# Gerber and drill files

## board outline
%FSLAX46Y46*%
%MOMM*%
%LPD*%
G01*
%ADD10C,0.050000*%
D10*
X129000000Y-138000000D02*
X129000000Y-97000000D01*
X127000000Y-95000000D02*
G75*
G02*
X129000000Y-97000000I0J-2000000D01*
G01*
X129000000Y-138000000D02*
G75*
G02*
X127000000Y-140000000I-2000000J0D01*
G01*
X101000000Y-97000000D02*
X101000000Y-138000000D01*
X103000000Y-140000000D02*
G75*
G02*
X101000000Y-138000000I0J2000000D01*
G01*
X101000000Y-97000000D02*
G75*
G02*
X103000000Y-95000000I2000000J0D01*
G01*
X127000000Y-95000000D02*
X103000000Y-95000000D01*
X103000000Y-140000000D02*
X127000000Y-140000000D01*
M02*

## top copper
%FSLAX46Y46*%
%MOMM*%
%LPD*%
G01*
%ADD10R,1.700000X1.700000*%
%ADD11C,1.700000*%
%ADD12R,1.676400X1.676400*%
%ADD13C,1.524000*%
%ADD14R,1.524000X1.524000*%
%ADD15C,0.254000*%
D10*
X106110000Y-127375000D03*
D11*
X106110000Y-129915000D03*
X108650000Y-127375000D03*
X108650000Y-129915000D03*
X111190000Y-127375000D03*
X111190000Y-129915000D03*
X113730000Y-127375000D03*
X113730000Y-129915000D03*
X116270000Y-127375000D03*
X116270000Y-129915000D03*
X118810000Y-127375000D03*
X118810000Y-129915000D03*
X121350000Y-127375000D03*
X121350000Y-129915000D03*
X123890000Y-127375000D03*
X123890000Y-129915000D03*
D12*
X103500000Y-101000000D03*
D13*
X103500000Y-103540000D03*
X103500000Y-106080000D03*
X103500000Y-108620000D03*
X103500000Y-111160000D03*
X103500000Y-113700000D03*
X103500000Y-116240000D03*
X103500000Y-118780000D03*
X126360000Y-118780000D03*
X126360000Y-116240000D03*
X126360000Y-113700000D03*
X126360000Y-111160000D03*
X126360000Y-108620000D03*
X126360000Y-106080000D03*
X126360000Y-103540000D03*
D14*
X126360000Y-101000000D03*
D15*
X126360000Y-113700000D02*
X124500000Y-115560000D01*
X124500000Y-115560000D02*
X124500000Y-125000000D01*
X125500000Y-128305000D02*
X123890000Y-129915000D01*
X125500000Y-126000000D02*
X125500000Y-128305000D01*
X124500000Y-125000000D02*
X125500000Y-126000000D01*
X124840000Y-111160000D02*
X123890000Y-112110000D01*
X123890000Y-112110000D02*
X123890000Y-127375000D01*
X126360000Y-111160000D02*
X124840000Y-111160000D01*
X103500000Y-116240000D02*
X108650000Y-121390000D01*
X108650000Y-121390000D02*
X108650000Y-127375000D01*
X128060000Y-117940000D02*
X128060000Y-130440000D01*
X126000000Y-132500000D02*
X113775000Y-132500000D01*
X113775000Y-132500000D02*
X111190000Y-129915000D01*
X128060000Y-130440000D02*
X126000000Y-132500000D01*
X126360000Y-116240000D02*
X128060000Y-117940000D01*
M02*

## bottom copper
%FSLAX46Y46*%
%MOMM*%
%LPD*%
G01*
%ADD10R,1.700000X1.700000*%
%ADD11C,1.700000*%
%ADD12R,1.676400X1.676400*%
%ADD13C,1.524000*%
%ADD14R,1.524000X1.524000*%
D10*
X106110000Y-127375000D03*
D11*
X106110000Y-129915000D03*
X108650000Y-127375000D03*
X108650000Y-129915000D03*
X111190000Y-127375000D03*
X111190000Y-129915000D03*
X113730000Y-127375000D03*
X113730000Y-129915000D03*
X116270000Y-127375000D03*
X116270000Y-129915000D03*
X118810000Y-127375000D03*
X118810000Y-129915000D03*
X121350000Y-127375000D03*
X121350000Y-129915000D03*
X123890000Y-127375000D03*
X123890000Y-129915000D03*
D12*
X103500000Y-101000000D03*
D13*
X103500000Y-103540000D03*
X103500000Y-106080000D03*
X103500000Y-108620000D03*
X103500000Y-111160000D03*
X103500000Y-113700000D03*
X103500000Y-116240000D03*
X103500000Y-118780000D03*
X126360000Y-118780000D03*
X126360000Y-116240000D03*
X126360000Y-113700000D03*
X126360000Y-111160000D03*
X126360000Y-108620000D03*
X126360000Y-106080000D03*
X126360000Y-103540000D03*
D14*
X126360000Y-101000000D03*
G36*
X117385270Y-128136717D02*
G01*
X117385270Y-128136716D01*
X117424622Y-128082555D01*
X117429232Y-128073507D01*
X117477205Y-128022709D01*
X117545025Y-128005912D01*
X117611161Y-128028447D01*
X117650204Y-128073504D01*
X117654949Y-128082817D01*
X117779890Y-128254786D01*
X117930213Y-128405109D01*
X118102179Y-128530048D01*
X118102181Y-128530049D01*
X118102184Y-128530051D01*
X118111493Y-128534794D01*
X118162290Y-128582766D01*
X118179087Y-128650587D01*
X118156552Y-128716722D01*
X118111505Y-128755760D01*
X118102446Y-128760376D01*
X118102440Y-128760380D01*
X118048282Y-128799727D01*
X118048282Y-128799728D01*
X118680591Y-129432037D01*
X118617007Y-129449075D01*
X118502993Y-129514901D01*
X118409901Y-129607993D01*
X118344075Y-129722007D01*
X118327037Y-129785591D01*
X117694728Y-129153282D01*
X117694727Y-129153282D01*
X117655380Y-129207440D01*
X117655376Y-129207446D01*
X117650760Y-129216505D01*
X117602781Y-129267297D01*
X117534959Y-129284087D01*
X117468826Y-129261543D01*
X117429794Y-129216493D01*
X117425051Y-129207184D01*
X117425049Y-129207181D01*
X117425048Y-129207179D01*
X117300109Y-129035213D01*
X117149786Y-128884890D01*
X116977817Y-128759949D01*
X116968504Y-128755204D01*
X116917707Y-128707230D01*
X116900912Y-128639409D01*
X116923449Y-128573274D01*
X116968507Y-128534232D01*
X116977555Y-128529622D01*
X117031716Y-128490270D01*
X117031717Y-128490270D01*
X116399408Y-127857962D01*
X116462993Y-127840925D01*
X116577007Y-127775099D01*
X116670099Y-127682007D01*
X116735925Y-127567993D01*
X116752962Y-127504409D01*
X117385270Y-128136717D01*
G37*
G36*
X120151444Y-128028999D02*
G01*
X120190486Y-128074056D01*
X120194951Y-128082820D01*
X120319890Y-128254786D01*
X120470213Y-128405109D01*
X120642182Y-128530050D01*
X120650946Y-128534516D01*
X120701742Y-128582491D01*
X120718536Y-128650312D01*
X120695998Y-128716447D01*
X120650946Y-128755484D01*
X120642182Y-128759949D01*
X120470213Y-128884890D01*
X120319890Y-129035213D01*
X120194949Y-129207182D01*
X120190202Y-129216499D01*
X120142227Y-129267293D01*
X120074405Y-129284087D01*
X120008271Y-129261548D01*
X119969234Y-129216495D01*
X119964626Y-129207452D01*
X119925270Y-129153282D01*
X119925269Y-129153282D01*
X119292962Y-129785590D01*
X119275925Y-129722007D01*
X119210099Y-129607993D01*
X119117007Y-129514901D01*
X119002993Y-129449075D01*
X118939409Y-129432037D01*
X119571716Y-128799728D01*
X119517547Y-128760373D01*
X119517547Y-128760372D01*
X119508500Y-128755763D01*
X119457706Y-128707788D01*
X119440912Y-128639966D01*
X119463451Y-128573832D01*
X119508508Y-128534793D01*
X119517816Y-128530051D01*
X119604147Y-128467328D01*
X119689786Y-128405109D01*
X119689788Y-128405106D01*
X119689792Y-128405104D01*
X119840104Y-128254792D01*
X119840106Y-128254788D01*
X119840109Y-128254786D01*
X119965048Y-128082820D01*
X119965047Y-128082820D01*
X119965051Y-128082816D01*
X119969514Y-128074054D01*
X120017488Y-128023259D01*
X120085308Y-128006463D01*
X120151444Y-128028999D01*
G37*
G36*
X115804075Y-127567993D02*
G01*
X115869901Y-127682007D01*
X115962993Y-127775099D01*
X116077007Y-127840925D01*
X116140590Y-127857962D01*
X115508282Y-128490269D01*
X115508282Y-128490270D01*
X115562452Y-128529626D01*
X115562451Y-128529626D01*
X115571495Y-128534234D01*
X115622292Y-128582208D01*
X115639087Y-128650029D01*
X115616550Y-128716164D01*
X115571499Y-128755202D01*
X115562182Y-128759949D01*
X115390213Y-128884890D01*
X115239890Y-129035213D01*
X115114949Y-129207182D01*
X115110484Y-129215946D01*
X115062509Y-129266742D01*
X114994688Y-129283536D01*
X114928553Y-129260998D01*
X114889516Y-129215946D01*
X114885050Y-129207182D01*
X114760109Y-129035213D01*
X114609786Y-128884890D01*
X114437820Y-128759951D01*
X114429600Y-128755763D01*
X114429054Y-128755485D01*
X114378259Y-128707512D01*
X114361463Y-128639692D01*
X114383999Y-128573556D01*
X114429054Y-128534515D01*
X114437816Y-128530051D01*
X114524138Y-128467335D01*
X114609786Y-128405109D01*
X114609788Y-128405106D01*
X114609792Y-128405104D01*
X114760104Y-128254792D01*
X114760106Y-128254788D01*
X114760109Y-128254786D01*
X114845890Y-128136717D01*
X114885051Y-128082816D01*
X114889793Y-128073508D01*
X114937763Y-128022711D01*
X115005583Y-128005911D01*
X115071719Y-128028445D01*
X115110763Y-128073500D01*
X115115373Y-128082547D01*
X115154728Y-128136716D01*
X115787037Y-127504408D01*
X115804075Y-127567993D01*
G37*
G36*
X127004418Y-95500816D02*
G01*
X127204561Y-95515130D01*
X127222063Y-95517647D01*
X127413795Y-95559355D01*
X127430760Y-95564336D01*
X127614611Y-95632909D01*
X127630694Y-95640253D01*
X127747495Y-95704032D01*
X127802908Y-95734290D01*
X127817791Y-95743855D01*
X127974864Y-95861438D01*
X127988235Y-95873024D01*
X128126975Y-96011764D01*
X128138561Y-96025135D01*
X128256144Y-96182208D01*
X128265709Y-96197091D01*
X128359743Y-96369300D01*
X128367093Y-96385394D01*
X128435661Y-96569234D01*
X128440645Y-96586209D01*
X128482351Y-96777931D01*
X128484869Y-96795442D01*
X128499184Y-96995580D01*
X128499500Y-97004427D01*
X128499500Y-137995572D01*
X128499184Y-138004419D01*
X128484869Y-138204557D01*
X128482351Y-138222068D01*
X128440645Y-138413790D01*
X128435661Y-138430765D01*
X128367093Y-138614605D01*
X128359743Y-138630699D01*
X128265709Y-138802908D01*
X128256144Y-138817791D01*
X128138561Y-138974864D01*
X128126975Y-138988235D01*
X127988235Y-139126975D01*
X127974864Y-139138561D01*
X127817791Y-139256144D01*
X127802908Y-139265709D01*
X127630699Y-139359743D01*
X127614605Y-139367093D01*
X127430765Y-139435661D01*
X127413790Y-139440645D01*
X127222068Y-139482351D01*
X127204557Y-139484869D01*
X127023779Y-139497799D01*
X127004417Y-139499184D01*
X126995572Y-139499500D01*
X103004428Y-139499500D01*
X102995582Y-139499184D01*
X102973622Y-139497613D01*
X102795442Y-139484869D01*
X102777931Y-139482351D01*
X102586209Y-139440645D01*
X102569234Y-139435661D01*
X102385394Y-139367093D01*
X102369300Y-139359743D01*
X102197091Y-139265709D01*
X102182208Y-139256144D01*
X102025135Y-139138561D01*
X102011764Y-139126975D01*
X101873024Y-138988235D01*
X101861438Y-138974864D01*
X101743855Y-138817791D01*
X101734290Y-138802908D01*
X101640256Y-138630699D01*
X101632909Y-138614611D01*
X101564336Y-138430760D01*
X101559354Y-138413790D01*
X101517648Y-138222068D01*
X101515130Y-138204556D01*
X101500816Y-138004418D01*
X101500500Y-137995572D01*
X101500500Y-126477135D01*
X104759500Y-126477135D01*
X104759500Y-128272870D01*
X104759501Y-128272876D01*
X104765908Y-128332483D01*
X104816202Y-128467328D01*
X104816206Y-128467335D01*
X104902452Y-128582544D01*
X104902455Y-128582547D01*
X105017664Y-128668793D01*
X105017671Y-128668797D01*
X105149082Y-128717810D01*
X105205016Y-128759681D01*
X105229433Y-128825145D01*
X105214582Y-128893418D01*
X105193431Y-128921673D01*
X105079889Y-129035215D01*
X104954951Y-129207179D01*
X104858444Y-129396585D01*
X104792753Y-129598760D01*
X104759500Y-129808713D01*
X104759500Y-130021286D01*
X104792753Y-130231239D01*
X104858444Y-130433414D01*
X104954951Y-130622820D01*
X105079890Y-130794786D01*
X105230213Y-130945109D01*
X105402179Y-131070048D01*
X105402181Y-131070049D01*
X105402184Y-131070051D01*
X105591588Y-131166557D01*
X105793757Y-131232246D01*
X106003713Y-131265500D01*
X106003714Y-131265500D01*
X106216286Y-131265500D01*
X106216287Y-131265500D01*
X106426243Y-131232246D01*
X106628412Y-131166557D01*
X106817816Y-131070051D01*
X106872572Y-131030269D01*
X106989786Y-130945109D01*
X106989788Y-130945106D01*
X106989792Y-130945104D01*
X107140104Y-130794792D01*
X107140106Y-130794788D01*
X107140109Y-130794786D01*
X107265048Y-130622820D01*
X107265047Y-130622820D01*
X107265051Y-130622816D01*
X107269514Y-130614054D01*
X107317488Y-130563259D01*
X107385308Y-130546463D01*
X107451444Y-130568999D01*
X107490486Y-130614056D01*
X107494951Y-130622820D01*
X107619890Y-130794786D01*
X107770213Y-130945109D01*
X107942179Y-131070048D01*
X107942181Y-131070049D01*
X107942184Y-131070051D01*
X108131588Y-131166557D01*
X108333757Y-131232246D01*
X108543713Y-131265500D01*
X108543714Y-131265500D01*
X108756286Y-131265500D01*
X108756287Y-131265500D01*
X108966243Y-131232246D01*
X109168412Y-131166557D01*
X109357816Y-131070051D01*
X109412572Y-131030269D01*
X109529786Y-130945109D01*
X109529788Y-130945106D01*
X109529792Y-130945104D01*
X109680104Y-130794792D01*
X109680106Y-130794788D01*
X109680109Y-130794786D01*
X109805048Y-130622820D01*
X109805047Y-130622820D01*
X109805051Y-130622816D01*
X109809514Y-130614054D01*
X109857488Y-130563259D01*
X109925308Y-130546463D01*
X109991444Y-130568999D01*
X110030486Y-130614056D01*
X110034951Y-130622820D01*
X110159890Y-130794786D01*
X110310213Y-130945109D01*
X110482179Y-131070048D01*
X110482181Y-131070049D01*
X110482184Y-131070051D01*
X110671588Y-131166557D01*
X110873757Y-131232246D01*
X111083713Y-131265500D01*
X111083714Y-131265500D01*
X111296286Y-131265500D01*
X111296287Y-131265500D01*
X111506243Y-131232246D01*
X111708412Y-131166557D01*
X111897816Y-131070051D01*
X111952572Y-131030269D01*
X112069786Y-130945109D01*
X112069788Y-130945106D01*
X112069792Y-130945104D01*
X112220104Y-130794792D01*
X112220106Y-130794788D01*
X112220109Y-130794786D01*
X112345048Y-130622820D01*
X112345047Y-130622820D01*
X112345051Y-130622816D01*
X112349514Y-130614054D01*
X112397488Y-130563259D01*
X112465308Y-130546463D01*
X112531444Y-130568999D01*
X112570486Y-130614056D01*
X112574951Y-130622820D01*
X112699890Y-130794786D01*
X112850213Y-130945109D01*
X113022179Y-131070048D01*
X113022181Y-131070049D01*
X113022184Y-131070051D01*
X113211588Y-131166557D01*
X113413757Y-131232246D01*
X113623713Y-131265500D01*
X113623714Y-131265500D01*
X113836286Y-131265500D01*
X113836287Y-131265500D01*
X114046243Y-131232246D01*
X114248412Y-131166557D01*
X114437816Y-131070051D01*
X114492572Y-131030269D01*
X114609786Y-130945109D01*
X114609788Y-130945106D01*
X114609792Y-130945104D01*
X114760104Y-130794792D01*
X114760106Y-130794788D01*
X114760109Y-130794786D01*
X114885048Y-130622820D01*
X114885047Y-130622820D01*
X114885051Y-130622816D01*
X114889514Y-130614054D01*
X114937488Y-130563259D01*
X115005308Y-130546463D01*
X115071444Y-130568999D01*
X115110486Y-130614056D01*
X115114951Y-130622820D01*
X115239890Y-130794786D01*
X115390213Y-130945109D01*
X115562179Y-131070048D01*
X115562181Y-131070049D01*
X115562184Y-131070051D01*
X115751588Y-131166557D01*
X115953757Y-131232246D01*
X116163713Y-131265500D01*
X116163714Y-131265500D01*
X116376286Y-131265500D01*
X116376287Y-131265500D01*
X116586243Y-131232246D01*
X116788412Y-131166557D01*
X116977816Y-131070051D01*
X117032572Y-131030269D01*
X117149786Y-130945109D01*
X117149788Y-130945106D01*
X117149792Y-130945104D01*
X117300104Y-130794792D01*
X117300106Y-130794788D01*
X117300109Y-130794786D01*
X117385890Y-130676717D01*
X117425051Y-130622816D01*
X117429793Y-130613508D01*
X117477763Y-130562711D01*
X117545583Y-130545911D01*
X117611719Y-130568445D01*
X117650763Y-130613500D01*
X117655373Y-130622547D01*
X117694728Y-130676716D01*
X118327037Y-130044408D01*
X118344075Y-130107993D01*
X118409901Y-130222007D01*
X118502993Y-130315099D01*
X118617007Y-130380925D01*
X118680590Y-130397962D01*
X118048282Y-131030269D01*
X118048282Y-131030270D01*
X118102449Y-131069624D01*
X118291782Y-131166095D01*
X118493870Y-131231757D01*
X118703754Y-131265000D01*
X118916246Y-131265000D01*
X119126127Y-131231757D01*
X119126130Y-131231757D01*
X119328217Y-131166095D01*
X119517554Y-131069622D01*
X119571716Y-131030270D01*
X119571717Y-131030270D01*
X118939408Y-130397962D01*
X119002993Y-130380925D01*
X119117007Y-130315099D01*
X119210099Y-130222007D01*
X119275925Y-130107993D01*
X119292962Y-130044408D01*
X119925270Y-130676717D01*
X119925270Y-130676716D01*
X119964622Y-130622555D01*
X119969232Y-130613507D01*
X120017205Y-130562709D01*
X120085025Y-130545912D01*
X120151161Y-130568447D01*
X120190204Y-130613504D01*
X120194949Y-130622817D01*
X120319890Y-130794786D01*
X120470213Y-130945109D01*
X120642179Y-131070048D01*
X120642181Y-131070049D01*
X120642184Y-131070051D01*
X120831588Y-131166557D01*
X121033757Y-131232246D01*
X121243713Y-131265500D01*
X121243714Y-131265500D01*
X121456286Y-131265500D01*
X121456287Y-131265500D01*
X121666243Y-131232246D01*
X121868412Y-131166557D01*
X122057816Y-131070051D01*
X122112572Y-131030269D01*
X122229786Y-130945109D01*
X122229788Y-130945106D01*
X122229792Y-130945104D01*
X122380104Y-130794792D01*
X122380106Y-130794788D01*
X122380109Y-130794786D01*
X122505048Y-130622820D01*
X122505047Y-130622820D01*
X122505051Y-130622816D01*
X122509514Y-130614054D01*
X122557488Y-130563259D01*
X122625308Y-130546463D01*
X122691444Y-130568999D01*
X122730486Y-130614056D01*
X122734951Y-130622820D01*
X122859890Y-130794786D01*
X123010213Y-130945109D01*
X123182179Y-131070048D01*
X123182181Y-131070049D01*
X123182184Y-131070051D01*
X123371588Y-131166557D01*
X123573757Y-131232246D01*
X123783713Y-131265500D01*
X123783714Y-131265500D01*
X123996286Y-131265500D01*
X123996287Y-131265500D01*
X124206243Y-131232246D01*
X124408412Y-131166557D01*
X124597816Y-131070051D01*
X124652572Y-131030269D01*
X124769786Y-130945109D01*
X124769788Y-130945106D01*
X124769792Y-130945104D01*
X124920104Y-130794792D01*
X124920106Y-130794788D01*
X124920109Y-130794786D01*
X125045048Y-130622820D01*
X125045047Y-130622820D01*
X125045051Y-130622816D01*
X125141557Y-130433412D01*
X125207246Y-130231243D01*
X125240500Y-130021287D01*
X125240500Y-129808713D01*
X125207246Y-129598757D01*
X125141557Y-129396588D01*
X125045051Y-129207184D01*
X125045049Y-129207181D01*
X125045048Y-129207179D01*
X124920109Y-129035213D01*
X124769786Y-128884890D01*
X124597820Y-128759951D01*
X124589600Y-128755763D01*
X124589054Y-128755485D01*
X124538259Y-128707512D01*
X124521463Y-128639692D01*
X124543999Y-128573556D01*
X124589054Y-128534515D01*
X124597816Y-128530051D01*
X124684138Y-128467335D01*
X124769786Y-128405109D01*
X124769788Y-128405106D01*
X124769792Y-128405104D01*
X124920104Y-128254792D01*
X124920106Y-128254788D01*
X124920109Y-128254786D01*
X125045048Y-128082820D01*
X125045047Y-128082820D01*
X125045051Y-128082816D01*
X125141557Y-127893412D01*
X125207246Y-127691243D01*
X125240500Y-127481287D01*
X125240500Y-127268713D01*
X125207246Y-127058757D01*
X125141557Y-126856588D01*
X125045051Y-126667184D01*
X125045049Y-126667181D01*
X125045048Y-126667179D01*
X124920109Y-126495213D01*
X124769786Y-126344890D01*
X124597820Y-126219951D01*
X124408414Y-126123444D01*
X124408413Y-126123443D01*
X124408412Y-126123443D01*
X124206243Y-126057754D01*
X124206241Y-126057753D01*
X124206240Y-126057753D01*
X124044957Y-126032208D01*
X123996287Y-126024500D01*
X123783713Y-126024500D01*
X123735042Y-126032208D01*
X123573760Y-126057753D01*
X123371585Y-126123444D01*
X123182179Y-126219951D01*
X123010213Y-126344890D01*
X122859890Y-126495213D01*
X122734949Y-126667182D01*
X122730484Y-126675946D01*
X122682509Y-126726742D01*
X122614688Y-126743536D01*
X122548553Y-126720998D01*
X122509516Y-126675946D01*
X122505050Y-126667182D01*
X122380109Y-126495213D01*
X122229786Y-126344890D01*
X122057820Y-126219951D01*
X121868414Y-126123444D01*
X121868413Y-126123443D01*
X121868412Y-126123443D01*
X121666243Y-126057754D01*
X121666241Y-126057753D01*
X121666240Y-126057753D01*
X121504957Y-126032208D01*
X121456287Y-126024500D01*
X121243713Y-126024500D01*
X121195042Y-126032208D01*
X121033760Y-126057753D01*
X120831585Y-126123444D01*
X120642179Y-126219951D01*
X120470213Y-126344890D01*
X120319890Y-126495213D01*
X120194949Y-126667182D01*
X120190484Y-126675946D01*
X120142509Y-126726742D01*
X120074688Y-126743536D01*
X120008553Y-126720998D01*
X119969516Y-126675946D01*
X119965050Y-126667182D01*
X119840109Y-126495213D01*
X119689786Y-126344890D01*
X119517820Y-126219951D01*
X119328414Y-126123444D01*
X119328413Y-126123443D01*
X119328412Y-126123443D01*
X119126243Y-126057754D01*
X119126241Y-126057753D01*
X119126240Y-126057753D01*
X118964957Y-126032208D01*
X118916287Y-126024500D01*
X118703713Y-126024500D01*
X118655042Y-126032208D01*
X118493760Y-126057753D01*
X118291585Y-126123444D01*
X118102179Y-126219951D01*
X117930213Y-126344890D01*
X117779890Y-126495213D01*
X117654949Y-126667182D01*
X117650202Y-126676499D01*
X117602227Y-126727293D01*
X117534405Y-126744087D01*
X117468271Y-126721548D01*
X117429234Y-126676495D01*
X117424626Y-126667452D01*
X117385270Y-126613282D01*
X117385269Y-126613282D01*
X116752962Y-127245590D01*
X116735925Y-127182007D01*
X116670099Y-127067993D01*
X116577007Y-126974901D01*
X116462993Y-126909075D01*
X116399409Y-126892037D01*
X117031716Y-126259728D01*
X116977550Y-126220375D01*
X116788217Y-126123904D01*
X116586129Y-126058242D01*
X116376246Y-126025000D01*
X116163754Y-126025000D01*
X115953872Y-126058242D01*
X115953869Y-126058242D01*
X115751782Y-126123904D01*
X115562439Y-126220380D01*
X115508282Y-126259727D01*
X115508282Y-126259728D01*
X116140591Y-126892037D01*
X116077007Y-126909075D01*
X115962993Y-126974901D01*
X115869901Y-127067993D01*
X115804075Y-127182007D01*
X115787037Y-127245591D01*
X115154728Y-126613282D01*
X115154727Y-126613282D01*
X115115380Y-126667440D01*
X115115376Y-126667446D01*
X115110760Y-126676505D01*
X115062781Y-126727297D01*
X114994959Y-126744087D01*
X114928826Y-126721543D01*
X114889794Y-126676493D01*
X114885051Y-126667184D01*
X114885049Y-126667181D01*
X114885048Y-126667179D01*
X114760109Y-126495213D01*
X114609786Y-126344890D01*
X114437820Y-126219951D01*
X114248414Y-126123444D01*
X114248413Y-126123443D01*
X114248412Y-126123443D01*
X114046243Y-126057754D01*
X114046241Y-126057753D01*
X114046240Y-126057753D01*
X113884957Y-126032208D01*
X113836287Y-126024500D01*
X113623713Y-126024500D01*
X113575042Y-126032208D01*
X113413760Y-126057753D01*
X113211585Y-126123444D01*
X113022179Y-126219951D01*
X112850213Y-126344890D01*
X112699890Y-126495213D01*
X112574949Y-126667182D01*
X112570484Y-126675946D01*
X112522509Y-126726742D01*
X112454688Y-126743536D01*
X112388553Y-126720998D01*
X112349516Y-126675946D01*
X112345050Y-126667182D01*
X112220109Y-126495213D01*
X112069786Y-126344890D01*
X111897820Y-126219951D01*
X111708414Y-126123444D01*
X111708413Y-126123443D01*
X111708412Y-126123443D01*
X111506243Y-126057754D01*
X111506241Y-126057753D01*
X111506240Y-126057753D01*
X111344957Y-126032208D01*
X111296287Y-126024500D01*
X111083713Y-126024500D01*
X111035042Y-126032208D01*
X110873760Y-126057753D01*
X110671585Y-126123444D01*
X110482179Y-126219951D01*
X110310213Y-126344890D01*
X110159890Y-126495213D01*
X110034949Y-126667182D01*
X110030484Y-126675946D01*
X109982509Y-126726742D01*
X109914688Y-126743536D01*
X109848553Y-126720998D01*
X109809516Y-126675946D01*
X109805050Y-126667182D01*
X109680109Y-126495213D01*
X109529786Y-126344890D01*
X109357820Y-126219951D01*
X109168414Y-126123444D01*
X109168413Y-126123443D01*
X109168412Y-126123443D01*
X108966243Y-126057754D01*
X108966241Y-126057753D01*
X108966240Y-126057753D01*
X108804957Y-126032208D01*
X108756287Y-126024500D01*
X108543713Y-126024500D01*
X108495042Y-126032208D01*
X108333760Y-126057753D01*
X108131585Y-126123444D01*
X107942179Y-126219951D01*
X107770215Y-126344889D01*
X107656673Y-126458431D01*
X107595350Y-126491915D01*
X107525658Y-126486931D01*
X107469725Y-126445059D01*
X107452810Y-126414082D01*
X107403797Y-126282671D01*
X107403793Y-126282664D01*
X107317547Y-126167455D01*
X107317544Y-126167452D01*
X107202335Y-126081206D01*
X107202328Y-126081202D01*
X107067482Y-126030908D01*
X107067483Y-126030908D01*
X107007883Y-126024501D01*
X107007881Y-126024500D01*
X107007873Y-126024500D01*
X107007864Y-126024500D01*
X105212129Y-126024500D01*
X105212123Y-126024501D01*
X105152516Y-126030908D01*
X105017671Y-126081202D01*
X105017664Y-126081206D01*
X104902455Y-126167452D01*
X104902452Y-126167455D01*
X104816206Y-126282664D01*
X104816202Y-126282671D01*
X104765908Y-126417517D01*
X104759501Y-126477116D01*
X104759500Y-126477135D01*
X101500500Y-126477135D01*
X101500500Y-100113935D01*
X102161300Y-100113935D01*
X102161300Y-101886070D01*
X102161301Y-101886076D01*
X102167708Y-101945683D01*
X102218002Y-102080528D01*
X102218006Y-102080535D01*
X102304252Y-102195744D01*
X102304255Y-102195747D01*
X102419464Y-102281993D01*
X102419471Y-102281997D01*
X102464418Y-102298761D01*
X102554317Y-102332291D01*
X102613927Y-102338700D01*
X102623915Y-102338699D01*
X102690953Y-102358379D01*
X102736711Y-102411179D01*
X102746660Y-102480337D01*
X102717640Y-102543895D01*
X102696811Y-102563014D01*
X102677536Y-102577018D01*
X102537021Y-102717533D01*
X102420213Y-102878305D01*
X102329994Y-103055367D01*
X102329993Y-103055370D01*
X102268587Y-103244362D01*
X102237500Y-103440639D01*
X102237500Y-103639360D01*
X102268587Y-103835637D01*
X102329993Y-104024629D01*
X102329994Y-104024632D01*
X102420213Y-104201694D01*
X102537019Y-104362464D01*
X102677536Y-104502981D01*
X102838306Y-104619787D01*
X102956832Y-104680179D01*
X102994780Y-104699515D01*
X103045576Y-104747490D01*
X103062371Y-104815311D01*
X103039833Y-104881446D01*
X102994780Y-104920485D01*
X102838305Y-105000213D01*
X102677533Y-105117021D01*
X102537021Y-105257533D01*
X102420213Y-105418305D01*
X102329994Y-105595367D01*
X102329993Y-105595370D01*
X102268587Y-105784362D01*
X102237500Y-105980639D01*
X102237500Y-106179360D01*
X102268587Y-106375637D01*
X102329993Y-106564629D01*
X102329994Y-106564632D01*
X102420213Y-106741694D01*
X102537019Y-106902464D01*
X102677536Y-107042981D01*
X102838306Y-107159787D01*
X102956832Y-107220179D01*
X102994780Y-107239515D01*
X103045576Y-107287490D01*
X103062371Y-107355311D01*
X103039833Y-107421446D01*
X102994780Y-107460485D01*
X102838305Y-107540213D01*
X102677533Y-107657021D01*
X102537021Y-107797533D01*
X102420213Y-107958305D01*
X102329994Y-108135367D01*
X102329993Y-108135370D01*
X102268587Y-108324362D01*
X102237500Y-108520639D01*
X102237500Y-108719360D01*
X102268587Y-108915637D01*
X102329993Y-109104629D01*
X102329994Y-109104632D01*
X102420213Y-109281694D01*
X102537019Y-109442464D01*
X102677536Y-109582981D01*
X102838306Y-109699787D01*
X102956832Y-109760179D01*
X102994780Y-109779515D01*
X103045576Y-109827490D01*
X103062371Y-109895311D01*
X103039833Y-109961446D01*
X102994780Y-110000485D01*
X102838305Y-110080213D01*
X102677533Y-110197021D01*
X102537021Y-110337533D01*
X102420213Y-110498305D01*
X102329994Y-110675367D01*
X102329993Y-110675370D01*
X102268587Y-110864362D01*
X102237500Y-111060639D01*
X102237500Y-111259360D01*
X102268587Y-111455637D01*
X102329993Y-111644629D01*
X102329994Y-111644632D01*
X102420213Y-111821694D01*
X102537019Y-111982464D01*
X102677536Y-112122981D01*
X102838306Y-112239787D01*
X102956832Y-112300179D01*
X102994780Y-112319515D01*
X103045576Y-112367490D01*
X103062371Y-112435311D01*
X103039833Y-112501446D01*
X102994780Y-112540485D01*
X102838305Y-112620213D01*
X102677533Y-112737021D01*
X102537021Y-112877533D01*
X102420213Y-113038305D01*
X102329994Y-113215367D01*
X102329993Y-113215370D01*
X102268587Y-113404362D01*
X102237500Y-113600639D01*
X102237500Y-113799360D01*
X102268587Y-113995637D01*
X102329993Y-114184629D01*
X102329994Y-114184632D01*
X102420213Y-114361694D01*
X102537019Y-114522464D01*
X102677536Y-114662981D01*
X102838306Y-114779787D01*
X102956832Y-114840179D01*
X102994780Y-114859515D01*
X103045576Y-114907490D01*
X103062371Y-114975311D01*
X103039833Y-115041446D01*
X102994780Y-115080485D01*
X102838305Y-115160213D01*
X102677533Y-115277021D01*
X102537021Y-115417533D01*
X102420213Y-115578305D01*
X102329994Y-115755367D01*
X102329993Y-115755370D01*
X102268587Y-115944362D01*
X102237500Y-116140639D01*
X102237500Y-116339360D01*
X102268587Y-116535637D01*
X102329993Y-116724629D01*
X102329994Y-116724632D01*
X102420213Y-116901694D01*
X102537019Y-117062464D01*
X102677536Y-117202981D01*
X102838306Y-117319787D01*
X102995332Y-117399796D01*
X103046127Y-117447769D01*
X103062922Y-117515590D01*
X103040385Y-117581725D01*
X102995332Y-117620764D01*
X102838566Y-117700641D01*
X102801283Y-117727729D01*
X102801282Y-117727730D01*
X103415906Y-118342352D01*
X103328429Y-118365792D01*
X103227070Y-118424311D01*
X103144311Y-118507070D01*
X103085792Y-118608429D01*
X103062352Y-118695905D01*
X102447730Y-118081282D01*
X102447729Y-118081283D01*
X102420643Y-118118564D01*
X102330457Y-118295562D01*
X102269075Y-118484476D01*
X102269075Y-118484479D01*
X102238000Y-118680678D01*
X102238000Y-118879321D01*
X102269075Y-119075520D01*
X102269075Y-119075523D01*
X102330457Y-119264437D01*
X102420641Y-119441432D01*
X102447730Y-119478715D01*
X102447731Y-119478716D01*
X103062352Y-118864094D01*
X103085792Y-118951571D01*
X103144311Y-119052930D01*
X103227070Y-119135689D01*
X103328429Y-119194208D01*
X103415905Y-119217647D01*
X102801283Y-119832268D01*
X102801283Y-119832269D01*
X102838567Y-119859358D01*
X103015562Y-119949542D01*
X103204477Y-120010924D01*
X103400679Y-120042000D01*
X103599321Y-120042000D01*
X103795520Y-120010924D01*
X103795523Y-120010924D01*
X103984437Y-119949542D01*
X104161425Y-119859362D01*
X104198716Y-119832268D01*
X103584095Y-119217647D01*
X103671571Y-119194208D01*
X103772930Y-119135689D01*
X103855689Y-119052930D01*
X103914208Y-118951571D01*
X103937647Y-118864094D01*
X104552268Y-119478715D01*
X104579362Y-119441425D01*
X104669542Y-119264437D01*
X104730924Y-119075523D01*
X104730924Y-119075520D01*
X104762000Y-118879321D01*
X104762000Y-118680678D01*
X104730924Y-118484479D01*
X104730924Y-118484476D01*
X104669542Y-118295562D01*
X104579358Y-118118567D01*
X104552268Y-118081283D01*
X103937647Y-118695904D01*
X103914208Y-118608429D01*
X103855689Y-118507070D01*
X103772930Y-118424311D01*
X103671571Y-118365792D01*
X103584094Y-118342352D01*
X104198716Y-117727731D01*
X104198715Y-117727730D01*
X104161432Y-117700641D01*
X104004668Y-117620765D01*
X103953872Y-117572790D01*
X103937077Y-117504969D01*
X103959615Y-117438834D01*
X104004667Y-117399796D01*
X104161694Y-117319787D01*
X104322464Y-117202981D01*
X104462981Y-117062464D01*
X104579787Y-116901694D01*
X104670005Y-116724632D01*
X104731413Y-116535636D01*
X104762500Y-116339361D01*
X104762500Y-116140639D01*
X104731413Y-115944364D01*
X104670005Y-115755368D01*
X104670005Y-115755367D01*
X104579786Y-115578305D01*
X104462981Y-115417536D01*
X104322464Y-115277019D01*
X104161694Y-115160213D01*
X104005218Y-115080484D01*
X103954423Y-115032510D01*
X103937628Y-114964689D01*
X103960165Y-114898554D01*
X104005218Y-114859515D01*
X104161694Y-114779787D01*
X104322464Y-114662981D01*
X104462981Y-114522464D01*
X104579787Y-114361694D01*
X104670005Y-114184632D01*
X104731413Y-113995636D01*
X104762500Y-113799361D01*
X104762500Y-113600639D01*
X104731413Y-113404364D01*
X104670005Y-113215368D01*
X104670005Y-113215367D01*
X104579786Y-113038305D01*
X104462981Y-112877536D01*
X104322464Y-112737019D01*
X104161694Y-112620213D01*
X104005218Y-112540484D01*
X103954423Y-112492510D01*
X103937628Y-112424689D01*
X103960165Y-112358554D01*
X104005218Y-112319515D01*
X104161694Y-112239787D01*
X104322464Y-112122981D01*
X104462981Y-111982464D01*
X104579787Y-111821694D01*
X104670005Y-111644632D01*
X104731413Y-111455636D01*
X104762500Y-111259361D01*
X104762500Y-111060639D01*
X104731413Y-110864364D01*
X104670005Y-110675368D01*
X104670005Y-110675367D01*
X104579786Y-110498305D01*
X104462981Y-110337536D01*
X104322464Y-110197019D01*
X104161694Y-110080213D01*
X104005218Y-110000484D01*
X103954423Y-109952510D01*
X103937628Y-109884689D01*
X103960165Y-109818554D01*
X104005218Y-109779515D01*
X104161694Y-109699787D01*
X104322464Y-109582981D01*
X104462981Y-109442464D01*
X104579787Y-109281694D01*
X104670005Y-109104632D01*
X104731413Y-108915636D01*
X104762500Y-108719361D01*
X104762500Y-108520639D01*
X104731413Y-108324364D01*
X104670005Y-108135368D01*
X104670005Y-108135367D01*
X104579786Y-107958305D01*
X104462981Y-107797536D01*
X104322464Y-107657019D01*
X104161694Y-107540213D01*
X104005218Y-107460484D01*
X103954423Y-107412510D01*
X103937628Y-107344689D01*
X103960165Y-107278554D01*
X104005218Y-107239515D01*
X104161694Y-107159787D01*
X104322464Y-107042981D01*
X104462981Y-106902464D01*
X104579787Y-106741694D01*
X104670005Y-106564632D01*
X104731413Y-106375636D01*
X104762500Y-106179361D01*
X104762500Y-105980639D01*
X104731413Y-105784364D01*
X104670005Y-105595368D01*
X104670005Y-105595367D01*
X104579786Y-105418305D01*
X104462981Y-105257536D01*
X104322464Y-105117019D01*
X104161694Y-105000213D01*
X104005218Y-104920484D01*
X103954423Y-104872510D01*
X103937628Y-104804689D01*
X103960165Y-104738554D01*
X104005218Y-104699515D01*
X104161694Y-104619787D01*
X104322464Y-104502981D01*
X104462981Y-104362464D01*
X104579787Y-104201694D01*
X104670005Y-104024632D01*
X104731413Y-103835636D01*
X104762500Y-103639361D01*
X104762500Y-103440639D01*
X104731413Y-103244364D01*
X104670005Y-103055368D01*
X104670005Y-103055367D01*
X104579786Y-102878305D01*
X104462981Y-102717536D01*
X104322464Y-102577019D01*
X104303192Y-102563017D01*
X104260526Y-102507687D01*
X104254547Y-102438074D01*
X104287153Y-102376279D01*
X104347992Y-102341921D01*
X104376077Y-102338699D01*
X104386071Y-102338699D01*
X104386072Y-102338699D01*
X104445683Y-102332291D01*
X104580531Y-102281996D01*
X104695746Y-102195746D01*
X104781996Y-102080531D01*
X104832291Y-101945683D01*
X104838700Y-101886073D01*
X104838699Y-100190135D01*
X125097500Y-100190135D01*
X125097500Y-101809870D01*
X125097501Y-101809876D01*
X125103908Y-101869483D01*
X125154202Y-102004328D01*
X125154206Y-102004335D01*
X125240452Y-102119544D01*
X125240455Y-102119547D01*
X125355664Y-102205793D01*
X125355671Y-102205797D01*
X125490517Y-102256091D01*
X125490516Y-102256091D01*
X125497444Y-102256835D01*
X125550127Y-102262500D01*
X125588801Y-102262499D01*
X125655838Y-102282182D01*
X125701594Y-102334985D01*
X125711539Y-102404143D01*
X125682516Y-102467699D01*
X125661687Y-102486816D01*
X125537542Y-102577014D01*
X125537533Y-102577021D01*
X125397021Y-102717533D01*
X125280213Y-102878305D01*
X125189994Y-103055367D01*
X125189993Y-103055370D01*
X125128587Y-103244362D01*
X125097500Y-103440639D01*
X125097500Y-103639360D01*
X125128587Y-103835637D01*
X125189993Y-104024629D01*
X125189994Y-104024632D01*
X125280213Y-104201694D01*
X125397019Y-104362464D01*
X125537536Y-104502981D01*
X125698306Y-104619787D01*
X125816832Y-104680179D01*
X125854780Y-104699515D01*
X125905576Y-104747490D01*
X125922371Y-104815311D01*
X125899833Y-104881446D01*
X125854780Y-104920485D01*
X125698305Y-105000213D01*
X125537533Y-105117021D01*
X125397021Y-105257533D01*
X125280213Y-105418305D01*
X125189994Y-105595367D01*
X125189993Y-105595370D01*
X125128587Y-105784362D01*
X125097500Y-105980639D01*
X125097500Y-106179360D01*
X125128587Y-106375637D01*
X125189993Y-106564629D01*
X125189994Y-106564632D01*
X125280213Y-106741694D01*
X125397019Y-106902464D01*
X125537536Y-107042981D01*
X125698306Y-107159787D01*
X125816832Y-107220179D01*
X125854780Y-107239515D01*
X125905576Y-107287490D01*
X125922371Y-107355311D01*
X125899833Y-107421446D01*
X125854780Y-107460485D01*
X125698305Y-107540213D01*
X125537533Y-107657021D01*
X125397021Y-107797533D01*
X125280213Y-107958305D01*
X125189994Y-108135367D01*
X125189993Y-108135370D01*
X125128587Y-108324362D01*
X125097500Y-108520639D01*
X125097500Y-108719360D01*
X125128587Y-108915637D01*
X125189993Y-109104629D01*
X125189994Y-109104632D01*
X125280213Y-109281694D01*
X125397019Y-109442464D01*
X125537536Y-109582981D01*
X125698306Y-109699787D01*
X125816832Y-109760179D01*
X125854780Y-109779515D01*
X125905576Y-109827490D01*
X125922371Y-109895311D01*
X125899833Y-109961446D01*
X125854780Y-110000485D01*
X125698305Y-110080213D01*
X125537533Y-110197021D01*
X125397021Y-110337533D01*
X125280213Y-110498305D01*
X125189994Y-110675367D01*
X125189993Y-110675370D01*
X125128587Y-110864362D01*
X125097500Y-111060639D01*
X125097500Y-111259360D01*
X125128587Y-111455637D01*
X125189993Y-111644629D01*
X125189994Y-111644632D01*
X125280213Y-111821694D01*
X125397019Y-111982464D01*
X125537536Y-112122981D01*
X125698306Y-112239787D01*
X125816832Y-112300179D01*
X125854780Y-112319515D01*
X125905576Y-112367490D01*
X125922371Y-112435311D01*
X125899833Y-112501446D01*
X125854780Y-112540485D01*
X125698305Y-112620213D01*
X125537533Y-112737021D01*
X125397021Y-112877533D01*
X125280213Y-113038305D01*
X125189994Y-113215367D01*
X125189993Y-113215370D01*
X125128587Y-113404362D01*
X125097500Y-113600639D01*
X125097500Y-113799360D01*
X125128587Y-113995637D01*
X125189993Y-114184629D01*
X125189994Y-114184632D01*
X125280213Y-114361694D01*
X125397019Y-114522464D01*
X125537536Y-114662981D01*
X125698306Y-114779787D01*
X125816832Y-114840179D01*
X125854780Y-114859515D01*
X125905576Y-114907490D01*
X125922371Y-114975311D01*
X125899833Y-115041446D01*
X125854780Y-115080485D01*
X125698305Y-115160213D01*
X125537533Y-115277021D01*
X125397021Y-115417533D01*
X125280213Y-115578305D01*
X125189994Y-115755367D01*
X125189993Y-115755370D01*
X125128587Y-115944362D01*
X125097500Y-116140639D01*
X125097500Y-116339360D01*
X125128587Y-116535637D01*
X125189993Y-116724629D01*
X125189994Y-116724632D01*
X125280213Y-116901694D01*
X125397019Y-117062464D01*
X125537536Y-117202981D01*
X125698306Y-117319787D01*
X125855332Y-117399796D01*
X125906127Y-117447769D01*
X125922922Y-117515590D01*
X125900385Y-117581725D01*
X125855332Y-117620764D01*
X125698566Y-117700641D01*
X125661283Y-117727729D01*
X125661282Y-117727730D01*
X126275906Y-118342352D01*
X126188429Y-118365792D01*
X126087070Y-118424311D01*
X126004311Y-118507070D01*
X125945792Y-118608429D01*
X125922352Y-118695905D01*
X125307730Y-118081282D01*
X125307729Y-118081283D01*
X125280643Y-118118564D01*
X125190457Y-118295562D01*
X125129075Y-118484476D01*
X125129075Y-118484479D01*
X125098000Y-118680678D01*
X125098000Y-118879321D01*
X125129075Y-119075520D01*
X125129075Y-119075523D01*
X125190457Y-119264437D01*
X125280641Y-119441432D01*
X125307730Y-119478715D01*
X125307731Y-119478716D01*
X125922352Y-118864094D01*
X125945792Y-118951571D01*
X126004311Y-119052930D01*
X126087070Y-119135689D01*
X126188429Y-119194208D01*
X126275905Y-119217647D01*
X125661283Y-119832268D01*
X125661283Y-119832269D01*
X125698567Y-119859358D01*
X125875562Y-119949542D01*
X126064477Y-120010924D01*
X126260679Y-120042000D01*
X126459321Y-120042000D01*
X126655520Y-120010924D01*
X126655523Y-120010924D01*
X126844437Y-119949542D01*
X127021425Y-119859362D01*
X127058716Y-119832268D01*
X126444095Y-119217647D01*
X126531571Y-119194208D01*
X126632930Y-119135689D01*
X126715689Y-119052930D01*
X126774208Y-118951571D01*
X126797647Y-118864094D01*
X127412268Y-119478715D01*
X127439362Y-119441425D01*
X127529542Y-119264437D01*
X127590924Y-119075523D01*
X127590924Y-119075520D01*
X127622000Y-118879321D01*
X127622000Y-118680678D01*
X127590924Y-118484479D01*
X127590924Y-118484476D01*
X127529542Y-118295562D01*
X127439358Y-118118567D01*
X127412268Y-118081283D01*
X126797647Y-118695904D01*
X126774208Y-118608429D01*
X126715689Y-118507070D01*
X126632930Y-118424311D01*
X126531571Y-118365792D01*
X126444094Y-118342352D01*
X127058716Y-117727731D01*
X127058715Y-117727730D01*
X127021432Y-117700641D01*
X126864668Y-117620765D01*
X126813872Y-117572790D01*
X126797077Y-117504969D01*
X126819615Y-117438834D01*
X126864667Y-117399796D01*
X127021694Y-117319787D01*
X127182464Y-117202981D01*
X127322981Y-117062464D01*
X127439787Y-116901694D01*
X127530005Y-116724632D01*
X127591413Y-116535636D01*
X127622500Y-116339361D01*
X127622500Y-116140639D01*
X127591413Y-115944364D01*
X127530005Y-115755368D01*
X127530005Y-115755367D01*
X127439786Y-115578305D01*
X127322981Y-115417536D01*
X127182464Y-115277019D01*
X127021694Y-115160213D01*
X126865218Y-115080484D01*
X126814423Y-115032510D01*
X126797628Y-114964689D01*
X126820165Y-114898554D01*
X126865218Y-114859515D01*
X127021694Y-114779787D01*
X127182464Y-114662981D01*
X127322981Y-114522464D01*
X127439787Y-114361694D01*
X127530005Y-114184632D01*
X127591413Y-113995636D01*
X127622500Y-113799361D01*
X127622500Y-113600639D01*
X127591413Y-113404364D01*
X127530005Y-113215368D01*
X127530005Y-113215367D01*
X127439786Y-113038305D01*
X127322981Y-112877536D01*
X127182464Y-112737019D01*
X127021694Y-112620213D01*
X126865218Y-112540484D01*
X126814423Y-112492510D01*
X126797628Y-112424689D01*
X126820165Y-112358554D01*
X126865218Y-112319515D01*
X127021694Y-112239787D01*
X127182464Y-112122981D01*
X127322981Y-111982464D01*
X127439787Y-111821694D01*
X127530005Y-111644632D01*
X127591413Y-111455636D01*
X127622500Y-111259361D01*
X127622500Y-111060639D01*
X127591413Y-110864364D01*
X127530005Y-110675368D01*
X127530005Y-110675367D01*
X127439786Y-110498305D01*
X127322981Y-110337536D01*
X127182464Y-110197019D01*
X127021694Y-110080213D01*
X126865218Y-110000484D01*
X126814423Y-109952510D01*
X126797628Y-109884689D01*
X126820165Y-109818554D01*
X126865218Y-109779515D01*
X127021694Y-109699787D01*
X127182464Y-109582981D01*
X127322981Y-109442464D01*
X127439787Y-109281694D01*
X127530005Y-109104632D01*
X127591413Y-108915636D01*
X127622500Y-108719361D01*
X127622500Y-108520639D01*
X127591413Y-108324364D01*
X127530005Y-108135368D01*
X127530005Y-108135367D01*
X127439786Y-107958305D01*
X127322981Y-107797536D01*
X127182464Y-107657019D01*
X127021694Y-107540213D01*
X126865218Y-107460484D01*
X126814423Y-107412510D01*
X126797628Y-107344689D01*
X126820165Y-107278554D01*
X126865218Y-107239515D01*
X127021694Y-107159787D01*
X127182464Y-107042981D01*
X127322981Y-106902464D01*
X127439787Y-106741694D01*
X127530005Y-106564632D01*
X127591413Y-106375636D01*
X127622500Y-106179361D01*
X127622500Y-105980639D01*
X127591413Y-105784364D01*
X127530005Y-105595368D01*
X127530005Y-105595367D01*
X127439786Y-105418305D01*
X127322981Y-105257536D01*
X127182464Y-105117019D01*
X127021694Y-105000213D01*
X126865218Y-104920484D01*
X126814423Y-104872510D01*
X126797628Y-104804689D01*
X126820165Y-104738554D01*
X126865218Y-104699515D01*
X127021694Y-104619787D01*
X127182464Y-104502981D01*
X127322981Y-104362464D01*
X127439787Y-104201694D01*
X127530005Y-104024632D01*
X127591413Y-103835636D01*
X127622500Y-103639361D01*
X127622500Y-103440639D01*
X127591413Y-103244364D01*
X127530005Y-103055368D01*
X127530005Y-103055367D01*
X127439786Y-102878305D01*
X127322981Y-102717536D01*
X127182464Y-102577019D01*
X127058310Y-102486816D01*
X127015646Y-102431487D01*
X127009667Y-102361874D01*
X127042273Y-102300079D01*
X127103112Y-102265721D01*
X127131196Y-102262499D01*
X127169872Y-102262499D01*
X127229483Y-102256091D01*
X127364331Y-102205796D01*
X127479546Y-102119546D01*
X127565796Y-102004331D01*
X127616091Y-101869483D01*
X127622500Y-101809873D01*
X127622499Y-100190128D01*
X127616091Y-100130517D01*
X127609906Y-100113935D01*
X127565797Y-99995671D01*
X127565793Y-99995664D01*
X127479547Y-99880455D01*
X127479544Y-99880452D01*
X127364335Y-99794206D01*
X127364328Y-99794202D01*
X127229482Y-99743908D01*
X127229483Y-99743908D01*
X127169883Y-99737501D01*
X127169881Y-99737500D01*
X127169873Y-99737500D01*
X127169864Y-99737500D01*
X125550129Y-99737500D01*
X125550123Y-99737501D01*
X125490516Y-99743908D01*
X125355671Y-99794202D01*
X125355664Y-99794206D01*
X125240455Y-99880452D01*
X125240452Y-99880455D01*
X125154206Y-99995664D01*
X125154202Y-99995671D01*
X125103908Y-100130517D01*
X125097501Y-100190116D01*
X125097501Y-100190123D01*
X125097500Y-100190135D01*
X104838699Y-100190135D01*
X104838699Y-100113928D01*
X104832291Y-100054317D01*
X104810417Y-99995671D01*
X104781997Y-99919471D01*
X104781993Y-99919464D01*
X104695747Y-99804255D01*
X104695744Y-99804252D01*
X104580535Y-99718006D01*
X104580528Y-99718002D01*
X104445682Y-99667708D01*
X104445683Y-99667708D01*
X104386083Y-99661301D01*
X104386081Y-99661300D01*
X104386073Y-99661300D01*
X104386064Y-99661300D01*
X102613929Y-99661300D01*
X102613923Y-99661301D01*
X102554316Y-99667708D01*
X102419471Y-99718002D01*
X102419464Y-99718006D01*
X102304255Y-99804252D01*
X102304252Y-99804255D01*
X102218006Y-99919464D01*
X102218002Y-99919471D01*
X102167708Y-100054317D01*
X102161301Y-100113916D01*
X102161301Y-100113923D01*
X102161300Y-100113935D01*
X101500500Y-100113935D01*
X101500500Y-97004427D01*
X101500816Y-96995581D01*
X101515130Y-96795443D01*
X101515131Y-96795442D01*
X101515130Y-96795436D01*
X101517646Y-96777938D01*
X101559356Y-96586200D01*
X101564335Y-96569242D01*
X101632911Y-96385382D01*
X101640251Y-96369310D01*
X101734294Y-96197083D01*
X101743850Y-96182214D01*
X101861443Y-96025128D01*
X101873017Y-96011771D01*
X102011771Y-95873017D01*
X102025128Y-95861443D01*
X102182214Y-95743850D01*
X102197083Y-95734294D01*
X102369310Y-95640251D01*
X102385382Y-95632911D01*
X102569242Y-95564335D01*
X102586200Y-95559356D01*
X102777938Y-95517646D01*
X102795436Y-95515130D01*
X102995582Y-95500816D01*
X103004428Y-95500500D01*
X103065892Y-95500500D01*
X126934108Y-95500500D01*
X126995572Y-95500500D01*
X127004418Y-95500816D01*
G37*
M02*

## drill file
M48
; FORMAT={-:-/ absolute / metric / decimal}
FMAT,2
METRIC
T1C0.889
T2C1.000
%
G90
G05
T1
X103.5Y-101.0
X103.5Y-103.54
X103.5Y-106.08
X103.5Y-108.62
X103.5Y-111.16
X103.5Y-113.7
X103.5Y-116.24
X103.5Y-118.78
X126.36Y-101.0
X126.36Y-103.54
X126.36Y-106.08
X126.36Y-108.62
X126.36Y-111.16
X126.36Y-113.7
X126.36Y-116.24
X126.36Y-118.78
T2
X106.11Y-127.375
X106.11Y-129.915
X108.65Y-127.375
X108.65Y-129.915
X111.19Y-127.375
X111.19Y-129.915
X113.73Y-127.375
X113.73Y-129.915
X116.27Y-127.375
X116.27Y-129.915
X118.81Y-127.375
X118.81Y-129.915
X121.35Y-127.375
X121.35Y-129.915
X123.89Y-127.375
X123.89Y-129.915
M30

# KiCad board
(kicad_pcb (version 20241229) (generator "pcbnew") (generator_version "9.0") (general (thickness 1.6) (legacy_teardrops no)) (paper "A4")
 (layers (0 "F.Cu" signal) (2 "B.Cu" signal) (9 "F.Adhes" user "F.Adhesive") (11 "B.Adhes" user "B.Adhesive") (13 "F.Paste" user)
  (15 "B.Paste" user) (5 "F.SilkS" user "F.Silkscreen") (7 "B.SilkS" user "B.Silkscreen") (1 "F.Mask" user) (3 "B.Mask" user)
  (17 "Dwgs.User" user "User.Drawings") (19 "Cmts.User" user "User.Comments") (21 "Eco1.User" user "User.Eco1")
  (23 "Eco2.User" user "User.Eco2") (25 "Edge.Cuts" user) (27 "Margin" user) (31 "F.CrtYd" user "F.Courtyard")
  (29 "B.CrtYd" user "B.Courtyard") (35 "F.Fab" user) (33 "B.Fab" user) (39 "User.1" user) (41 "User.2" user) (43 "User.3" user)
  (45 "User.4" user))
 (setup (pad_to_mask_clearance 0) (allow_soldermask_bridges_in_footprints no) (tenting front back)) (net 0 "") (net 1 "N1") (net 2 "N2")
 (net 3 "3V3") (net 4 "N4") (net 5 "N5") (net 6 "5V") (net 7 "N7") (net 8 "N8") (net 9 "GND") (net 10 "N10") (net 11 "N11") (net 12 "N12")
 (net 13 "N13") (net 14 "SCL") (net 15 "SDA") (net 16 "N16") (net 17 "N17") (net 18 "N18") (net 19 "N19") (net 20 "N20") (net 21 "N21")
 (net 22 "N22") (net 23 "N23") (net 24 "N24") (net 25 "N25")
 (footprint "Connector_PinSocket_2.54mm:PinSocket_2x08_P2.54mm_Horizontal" (layer "F.Cu") (at 106.11 127.375 90)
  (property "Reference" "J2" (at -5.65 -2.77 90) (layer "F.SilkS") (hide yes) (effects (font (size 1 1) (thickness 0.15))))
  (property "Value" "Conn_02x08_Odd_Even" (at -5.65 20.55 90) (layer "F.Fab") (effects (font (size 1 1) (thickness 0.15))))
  (pad "1" thru_hole rect (at 0 0 90) (size 1.7 1.7) (drill 1) (layers "*.Cu" "*.Mask") (remove_unused_layers no) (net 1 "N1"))
  (pad "2" thru_hole circle (at -2.54 0 90) (size 1.7 1.7) (drill 1) (layers "*.Cu" "*.Mask") (remove_unused_layers no) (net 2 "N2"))
  (pad "3" thru_hole circle (at 0 2.54 90) (size 1.7 1.7) (drill 1) (layers "*.Cu" "*.Mask") (remove_unused_layers no) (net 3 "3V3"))
  (pad "4" thru_hole circle (at -2.54 2.54 90) (size 1.7 1.7) (drill 1) (layers "*.Cu" "*.Mask") (remove_unused_layers no) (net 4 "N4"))
  (pad "5" thru_hole circle (at 0 5.08 90) (size 1.7 1.7) (drill 1) (layers "*.Cu" "*.Mask") (remove_unused_layers no) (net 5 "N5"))
  (pad "6" thru_hole circle (at -2.54 5.08 90) (size 1.7 1.7) (drill 1) (layers "*.Cu" "*.Mask") (remove_unused_layers no) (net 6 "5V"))
  (pad "7" thru_hole circle (at 0 7.62 90) (size 1.7 1.7) (drill 1) (layers "*.Cu" "*.Mask") (remove_unused_layers no) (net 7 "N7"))
  (pad "8" thru_hole circle (at -2.54 7.62 90) (size 1.7 1.7) (drill 1) (layers "*.Cu" "*.Mask") (remove_unused_layers no) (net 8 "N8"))
  (pad "9" thru_hole circle (at 0 10.16 90) (size 1.7 1.7) (drill 1) (layers "*.Cu" "*.Mask") (remove_unused_layers no) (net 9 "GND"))
  (pad "10" thru_hole circle (at -2.54 10.16 90) (size 1.7 1.7) (drill 1) (layers "*.Cu" "*.Mask") (remove_unused_layers no) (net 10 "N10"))
  (pad "11" thru_hole circle (at 0 12.7 90) (size 1.7 1.7) (drill 1) (layers "*.Cu" "*.Mask") (remove_unused_layers no) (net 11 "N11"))
  (pad "12" thru_hole circle (at -2.54 12.7 90) (size 1.7 1.7) (drill 1) (layers "*.Cu" "*.Mask") (remove_unused_layers no) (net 9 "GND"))
  (pad "13" thru_hole circle (at 0 15.24 90) (size 1.7 1.7) (drill 1) (layers "*.Cu" "*.Mask") (remove_unused_layers no) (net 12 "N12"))
  (pad "14" thru_hole circle (at -2.54 15.24 90) (size 1.7 1.7) (drill 1) (layers "*.Cu" "*.Mask") (remove_unused_layers no) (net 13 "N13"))
  (pad "15" thru_hole circle (at 0 17.78 90) (size 1.7 1.7) (drill 1) (layers "*.Cu" "*.Mask") (remove_unused_layers no) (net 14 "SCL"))
  (pad "16" thru_hole circle (at -2.54 17.78 90) (size 1.7 1.7) (drill 1) (layers "*.Cu" "*.Mask") (remove_unused_layers no) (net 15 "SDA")))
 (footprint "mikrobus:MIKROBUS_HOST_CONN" (layer "F.Cu") (at 103.5 101)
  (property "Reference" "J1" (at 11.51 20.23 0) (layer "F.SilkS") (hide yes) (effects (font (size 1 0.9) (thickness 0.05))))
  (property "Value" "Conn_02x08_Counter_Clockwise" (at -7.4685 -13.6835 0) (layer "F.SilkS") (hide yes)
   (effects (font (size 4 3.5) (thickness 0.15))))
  (pad "1" thru_hole rect (at 0 0) (size 1.6764 1.6764) (drill 0.889) (layers "*.Cu" "*.Mask") (remove_unused_layers no) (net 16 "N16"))
  (pad "2" thru_hole circle (at 0 2.54) (size 1.524 1.524) (drill 0.889) (layers "*.Cu" "*.Mask") (remove_unused_layers no) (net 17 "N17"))
  (pad "3" thru_hole circle (at 0 5.08) (size 1.524 1.524) (drill 0.889) (layers "*.Cu" "*.Mask") (remove_unused_layers no) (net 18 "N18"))
  (pad "4" thru_hole circle (at 0 7.62) (size 1.524 1.524) (drill 0.889) (layers "*.Cu" "*.Mask") (remove_unused_layers no) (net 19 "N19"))
  (pad "5" thru_hole circle (at 0 10.16) (size 1.524 1.524) (drill 0.889) (layers "*.Cu" "*.Mask") (remove_unused_layers no) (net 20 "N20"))
  (pad "6" thru_hole circle (at 0 12.7) (size 1.524 1.524) (drill 0.889) (layers "*.Cu" "*.Mask") (remove_unused_layers no) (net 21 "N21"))
  (pad "7" thru_hole circle (at 0 15.24) (size 1.524 1.524) (drill 0.889) (layers "*.Cu" "*.Mask") (remove_unused_layers no) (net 3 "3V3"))
  (pad "8" thru_hole circle (at 0 17.78) (size 1.524 1.524) (drill 0.889) (layers "*.Cu" "*.Mask") (remove_unused_layers no) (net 9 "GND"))
  (pad "9" thru_hole circle (at 22.86 17.78) (size 1.524 1.524) (drill 0.889) (layers "*.Cu" "*.Mask") (remove_unused_layers no)
   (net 9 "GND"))
  (pad "10" thru_hole circle (at 22.86 15.24) (size 1.524 1.524) (drill 0.889) (layers "*.Cu" "*.Mask") (remove_unused_layers no)
   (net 6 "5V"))
  (pad "11" thru_hole circle (at 22.86 12.7) (size 1.524 1.524) (drill 0.889) (layers "*.Cu" "*.Mask") (remove_unused_layers no)
   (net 15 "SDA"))
  (pad "12" thru_hole circle (at 22.86 10.16) (size 1.524 1.524) (drill 0.889) (layers "*.Cu" "*.Mask") (remove_unused_layers no)
   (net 14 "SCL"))
  (pad "13" thru_hole circle (at 22.86 7.62) (size 1.524 1.524) (drill 0.889) (layers "*.Cu" "*.Mask") (remove_unused_layers no)
   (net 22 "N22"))
  (pad "14" thru_hole circle (at 22.86 5.08) (size 1.524 1.524) (drill 0.889) (layers "*.Cu" "*.Mask") (remove_unused_layers no)
   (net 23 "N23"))
  (pad "15" thru_hole circle (at 22.86 2.54) (size 1.524 1.524) (drill 0.889) (layers "*.Cu" "*.Mask") (remove_unused_layers no)
   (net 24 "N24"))
  (pad "16" thru_hole rect (at 22.86 0) (size 1.524 1.524) (drill 0.889) (layers "*.Cu" "*.Mask") (remove_unused_layers no) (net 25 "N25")))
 (gr_line (start 129 138) (end 129 97) (stroke (width 0.05) (type default)) (layer "Edge.Cuts"))
 (gr_arc (start 127 95) (mid 128.414214 95.585786) (end 129 97) (stroke (width 0.05) (type default)) (layer "Edge.Cuts"))
 (gr_arc (start 129 138) (mid 128.414214 139.414214) (end 127 140) (stroke (width 0.05) (type default)) (layer "Edge.Cuts"))
 (gr_line (start 101 97) (end 101 138) (stroke (width 0.05) (type default)) (layer "Edge.Cuts"))
 (gr_arc (start 103 140) (mid 101.585786 139.414214) (end 101 138) (stroke (width 0.05) (type default)) (layer "Edge.Cuts"))
 (gr_arc (start 101 97) (mid 101.585786 95.585786) (end 103 95) (stroke (width 0.05) (type default)) (layer "Edge.Cuts"))
 (gr_line (start 127 95) (end 103 95) (stroke (width 0.05) (type default)) (layer "Edge.Cuts"))
 (gr_line (start 103 140) (end 127 140) (stroke (width 0.05) (type default)) (layer "Edge.Cuts"))
 (segment (start 126.36 113.7) (end 124.5 115.56) (width 0.254) (layer "F.Cu") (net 15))
 (segment (start 124.5 115.56) (end 124.5 125) (width 0.254) (layer "F.Cu") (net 15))
 (segment (start 125.5 128.305) (end 123.89 129.915) (width 0.254) (layer "F.Cu") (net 15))
 (segment (start 125.5 126) (end 125.5 128.305) (width 0.254) (layer "F.Cu") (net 15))
 (segment (start 124.5 125) (end 125.5 126) (width 0.254) (layer "F.Cu") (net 15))
 (segment (start 124.84 111.16) (end 123.89 112.11) (width 0.254) (layer "F.Cu") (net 14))
 (segment (start 123.89 112.11) (end 123.89 127.375) (width 0.254) (layer "F.Cu") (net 14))
 (segment (start 126.36 111.16) (end 124.84 111.16) (width 0.254) (layer "F.Cu") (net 14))
 (segment (start 103.5 116.24) (end 108.65 121.39) (width 0.254) (layer "F.Cu") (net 3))
 (segment (start 108.65 121.39) (end 108.65 127.375) (width 0.254) (layer "F.Cu") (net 3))
 (segment (start 128.06 117.94) (end 128.06 130.44) (width 0.254) (layer "F.Cu") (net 6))
 (segment (start 126 132.5) (end 113.775 132.5) (width 0.254) (layer "F.Cu") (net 6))
 (segment (start 113.775 132.5) (end 111.19 129.915) (width 0.254) (layer "F.Cu") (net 6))
 (segment (start 128.06 130.44) (end 126 132.5) (width 0.254) (layer "F.Cu") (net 6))
 (segment (start 126.36 116.24) (end 128.06 117.94) (width 0.254) (layer "F.Cu") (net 6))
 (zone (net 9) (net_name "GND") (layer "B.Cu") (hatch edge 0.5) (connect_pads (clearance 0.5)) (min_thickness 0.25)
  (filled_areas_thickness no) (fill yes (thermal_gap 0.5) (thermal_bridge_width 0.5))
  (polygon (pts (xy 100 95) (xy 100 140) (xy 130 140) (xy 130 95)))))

